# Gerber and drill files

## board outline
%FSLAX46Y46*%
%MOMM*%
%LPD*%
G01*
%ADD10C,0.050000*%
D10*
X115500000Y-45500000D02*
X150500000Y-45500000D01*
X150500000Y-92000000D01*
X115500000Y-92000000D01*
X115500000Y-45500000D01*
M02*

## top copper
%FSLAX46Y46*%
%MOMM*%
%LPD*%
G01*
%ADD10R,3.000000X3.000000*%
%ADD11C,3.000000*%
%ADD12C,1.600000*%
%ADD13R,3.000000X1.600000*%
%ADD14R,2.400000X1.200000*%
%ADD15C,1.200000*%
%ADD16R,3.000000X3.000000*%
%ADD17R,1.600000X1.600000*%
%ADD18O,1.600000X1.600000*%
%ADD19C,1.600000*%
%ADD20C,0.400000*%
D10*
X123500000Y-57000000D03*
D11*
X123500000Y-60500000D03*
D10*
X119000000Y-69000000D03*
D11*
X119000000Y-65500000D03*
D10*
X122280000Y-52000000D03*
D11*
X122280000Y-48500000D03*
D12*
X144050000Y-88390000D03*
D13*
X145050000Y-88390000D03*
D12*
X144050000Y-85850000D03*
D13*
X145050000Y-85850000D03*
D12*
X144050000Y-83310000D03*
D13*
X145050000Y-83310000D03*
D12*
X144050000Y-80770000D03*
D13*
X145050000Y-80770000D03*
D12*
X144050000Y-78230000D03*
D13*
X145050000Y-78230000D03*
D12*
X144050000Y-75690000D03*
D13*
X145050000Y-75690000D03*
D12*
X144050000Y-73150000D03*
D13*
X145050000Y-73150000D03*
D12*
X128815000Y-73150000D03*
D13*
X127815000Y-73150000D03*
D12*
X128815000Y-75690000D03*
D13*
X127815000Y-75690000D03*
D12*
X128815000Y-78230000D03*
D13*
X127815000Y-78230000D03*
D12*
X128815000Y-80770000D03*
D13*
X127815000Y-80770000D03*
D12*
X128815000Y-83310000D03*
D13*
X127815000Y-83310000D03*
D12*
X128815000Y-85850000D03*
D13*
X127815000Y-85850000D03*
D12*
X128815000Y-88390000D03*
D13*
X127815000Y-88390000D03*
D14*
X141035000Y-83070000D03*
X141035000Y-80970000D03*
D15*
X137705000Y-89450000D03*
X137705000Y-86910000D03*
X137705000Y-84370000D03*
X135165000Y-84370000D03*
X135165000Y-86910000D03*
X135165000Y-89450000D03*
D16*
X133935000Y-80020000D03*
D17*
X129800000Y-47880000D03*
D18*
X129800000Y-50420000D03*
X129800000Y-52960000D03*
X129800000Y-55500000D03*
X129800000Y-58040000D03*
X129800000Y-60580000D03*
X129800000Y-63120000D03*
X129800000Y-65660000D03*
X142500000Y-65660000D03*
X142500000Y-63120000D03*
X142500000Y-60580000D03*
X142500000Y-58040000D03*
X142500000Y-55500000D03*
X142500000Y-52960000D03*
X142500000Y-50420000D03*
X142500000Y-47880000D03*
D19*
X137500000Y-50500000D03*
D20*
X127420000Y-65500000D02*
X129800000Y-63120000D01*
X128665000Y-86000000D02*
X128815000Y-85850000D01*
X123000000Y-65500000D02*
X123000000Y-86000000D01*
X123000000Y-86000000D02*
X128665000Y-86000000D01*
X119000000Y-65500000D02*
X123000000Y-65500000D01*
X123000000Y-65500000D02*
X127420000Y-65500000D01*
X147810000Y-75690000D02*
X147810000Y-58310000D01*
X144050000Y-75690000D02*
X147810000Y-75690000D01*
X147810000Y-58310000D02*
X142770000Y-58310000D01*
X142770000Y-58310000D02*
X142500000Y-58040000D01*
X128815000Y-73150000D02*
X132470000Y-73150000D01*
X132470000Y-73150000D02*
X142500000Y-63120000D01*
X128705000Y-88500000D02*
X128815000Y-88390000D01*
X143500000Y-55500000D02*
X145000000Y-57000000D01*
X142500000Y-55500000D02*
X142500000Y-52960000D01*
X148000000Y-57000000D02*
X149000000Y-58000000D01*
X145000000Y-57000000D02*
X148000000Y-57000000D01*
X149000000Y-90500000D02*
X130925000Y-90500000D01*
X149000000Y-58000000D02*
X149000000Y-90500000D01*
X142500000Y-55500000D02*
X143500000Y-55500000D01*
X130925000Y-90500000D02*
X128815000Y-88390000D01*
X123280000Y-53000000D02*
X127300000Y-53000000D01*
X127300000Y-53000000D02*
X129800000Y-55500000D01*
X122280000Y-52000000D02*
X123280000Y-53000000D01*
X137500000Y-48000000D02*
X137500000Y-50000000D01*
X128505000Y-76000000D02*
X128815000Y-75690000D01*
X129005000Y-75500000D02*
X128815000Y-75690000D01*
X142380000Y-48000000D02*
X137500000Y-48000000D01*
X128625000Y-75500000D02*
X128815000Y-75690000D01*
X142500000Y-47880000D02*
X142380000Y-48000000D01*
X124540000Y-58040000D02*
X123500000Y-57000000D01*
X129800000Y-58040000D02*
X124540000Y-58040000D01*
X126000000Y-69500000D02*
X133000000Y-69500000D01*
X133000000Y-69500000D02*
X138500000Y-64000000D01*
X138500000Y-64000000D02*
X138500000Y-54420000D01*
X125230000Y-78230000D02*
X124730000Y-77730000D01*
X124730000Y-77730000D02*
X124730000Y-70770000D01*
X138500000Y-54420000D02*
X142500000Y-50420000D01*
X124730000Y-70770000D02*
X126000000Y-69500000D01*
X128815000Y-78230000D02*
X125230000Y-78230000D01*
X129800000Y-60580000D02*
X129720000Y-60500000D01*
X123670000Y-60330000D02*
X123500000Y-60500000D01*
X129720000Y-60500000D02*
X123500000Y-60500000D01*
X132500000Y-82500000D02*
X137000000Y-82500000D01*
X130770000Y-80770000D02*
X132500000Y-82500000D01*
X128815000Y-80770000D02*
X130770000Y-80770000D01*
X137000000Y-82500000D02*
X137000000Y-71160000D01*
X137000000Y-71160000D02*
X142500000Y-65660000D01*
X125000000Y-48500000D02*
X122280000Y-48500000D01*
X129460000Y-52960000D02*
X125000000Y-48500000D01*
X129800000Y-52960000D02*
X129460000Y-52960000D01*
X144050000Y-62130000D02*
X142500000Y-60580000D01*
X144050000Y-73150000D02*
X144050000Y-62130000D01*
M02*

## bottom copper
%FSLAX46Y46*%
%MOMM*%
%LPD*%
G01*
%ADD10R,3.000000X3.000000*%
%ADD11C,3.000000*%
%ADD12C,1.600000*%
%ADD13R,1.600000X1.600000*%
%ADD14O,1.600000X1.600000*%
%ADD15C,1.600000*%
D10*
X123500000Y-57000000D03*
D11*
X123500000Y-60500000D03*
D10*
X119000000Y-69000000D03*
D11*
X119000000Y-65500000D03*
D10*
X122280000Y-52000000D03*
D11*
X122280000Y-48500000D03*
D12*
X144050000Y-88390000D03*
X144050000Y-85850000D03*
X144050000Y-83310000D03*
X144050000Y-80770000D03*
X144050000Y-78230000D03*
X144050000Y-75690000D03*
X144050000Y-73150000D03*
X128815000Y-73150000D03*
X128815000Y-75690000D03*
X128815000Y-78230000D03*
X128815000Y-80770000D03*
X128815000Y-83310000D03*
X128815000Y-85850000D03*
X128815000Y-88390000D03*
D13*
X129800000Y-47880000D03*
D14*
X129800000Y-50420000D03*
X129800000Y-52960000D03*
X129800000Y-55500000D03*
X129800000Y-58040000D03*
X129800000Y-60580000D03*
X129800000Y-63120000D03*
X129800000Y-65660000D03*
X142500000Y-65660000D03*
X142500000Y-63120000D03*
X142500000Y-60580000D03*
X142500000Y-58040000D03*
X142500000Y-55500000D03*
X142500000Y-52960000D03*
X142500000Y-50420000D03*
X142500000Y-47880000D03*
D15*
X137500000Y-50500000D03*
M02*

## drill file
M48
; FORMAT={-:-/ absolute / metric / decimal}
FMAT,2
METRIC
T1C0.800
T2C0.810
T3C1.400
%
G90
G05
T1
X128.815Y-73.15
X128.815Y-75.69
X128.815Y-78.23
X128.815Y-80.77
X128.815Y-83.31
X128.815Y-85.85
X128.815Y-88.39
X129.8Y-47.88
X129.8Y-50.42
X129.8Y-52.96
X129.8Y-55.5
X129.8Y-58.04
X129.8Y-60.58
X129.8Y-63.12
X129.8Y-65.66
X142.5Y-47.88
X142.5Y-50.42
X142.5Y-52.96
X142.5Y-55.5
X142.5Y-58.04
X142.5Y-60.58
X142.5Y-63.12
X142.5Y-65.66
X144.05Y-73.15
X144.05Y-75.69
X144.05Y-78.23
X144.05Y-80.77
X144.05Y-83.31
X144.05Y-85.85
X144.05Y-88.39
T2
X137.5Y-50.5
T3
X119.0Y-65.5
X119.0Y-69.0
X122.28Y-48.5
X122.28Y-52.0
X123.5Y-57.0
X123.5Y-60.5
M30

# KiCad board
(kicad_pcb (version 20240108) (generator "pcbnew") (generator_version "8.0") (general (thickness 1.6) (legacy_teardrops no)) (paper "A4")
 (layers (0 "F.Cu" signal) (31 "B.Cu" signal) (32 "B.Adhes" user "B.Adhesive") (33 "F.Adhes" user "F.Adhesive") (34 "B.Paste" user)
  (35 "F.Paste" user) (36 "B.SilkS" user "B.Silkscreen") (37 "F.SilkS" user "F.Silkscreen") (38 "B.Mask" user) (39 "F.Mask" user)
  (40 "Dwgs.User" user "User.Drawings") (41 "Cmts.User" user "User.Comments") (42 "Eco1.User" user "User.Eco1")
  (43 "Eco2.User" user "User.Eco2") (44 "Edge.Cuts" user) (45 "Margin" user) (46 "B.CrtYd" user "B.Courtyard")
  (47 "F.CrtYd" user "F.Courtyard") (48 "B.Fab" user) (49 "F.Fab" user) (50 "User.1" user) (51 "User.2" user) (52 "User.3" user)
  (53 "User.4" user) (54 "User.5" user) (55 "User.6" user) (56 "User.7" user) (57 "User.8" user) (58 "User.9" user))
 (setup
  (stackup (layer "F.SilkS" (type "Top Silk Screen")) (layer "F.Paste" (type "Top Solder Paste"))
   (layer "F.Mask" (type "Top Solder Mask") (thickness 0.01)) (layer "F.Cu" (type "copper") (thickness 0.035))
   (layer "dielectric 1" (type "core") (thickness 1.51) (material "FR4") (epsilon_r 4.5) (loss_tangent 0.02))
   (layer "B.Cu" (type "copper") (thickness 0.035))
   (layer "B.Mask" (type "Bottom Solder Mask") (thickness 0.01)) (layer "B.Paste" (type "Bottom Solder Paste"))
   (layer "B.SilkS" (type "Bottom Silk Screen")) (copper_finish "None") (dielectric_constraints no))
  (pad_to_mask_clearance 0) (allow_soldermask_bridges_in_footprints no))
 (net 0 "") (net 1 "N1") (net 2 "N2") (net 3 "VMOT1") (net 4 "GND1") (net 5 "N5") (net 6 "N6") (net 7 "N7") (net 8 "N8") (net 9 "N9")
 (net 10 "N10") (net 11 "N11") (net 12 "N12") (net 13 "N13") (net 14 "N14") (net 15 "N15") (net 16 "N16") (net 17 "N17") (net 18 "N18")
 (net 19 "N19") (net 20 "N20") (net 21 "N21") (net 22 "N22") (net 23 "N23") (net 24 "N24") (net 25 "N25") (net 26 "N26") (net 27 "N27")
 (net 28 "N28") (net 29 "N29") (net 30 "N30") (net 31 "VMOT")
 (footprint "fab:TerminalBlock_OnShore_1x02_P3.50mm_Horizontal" (layer "F.Cu") (at 123.5 57 -90)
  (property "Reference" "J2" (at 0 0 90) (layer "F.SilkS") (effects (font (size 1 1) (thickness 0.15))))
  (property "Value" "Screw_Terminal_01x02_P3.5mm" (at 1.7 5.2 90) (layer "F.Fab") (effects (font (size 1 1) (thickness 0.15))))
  (pad "1" thru_hole rect (at 0 0 270) (size 3 3) (drill 1.4) (layers "*.Cu" "*.Mask") (remove_unused_layers no) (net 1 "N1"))
  (pad "2" thru_hole circle (at 3.5 0 270) (size 3 3) (drill 1.4) (layers "*.Cu" "*.Mask") (remove_unused_layers no) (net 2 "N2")))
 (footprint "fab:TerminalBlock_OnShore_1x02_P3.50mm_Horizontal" (layer "F.Cu") (at 119 69 90)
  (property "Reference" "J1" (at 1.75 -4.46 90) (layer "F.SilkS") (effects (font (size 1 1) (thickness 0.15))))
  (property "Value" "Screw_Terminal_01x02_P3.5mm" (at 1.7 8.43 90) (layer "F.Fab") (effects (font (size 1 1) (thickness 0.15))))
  (pad "1" thru_hole rect (at 0 0 90) (size 3 3) (drill 1.4) (layers "*.Cu" "*.Mask") (remove_unused_layers no) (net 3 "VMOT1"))
  (pad "2" thru_hole circle (at 3.5 0 90) (size 3 3) (drill 1.4) (layers "*.Cu" "*.Mask") (remove_unused_layers no) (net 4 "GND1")))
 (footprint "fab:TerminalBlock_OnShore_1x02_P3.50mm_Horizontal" (layer "F.Cu") (at 122.28 52 90)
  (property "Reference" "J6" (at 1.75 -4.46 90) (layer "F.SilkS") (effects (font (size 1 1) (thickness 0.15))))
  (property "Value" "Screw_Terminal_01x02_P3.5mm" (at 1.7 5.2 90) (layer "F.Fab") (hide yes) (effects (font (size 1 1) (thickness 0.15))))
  (pad "1" thru_hole rect (at 0 0 90) (size 3 3) (drill 1.4) (layers "*.Cu" "*.Mask") (remove_unused_layers no) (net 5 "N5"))
  (pad "2" thru_hole circle (at 3.5 0 90) (size 3 3) (drill 1.4) (layers "*.Cu" "*.Mask") (remove_unused_layers no) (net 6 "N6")))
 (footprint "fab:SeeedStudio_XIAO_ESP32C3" (layer "F.Cu") (at 136.435 80.77 180)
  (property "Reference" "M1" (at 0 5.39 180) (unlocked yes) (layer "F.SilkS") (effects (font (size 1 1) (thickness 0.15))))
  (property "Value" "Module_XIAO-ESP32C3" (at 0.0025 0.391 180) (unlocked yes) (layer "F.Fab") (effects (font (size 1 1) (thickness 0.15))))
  (pad "1" thru_hole circle (at -7.615 -7.62 180) (size 1.6 1.6) (drill 0.8) (layers "*.Cu" "*.Mask") (remove_unused_layers no) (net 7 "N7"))
  (pad "1" smd rect (at -7.615 -7.62 180) (size 3 1.6) (drill (offset -1 0)) (layers "F.Cu" "F.Paste" "F.Mask") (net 7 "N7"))
  (pad "2" thru_hole circle (at -7.615 -5.08 180) (size 1.6 1.6) (drill 0.8) (layers "*.Cu" "*.Mask") (remove_unused_layers no) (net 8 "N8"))
  (pad "2" smd rect (at -7.615 -5.08 180) (size 3 1.6) (drill (offset -1 0)) (layers "F.Cu" "F.Paste" "F.Mask") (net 8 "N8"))
  (pad "3" thru_hole circle (at -7.615 -2.54 180) (size 1.6 1.6) (drill 0.8) (layers "*.Cu" "*.Mask") (remove_unused_layers no) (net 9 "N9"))
  (pad "3" smd rect (at -7.615 -2.54 180) (size 3 1.6) (drill (offset -1 0)) (layers "F.Cu" "F.Paste" "F.Mask") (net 9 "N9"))
  (pad "4" thru_hole circle (at -7.615 0 180) (size 1.6 1.6) (drill 0.8) (layers "*.Cu" "*.Mask") (remove_unused_layers no) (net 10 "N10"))
  (pad "4" smd rect (at -7.615 0 180) (size 3 1.6) (drill (offset -1 0)) (layers "F.Cu" "F.Paste" "F.Mask") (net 10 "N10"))
  (pad "5" thru_hole circle (at -7.615 2.54 180) (size 1.6 1.6) (drill 0.8) (layers "*.Cu" "*.Mask") (remove_unused_layers no)
   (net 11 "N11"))
  (pad "5" smd rect (at -7.615 2.54 180) (size 3 1.6) (drill (offset -1 0)) (layers "F.Cu" "F.Paste" "F.Mask") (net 11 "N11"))
  (pad "6" thru_hole circle (at -7.615 5.08 180) (size 1.6 1.6) (drill 0.8) (layers "*.Cu" "*.Mask") (remove_unused_layers no)
   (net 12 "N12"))
  (pad "6" smd rect (at -7.615 5.08 180) (size 3 1.6) (drill (offset -1 0)) (layers "F.Cu" "F.Paste" "F.Mask") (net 12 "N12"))
  (pad "7" thru_hole circle (at -7.615 7.62 180) (size 1.6 1.6) (drill 0.8) (layers "*.Cu" "*.Mask") (remove_unused_layers no)
   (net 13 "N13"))
  (pad "7" smd rect (at -7.615 7.62 180) (size 3 1.6) (drill (offset -1 0)) (layers "F.Cu" "F.Paste" "F.Mask") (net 13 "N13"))
  (pad "8" thru_hole circle (at 7.62 7.62 180) (size 1.6 1.6) (drill 0.8) (layers "*.Cu" "*.Mask") (remove_unused_layers no) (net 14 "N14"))
  (pad "8" smd rect (at 7.62 7.62 180) (size 3 1.6) (drill (offset 1 0)) (layers "F.Cu" "F.Paste" "F.Mask") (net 14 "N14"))
  (pad "9" thru_hole circle (at 7.62 5.08 180) (size 1.6 1.6) (drill 0.8) (layers "*.Cu" "*.Mask") (remove_unused_layers no) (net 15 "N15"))
  (pad "9" smd rect (at 7.62 5.08 180) (size 3 1.6) (drill (offset 1 0)) (layers "F.Cu" "F.Paste" "F.Mask") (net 15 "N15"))
  (pad "10" thru_hole circle (at 7.62 2.54 180) (size 1.6 1.6) (drill 0.8) (layers "*.Cu" "*.Mask") (remove_unused_layers no) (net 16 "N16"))
  (pad "10" smd rect (at 7.62 2.54 180) (size 3 1.6) (drill (offset 1 0)) (layers "F.Cu" "F.Paste" "F.Mask") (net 16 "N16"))
  (pad "11" thru_hole circle (at 7.62 0 180) (size 1.6 1.6) (drill 0.8) (layers "*.Cu" "*.Mask") (remove_unused_layers no) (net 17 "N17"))
  (pad "11" smd rect (at 7.62 0 180) (size 3 1.6) (drill (offset 1 0)) (layers "F.Cu" "F.Paste" "F.Mask") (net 17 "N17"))
  (pad "12" thru_hole circle (at 7.62 -2.54 180) (size 1.6 1.6) (drill 0.8) (layers "*.Cu" "*.Mask") (remove_unused_layers no)
   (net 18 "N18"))
  (pad "12" smd rect (at 7.62 -2.54 180) (size 3 1.6) (drill (offset 1 0)) (layers "F.Cu" "F.Paste" "F.Mask") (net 18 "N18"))
  (pad "13" thru_hole circle (at 7.62 -5.08 180) (size 1.6 1.6) (drill 0.8) (layers "*.Cu" "*.Mask") (remove_unused_layers no)
   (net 4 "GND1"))
  (pad "13" smd rect (at 7.62 -5.08 180) (size 3 1.6) (drill (offset 1 0)) (layers "F.Cu" "F.Paste" "F.Mask") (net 4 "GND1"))
  (pad "14" thru_hole circle (at 7.62 -7.62 180) (size 1.6 1.6) (drill 0.8) (layers "*.Cu" "*.Mask") (remove_unused_layers no)
   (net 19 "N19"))
  (pad "14" smd rect (at 7.62 -7.62 180) (size 3 1.6) (drill (offset 1 0)) (layers "F.Cu" "F.Paste" "F.Mask") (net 19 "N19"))
  (pad "15" smd rect (at -4.6 -2.3 180) (size 2.4 1.2) (layers "F.Cu" "F.Paste" "F.Mask") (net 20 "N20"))
  (pad "16" smd rect (at -4.6 -0.2 180) (size 2.4 1.2) (layers "F.Cu" "F.Paste" "F.Mask") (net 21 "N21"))
  (pad "17" smd circle (at -1.27 -8.68 180) (size 1.2 1.2) (layers "F.Cu" "F.Paste" "F.Mask") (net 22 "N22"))
  (pad "18" smd circle (at -1.27 -6.14 180) (size 1.2 1.2) (layers "F.Cu" "F.Paste" "F.Mask") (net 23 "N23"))
  (pad "19" smd circle (at -1.27 -3.6 180) (size 1.2 1.2) (layers "F.Cu" "F.Paste" "F.Mask") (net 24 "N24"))
  (pad "20" smd circle (at 1.27 -3.6 180) (size 1.2 1.2) (layers "F.Cu" "F.Paste" "F.Mask") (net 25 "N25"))
  (pad "21" smd circle (at 1.27 -6.14 180) (size 1.2 1.2) (layers "F.Cu" "F.Paste" "F.Mask") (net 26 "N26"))
  (pad "22" smd circle (at 1.27 -8.68 180) (size 1.2 1.2) (layers "F.Cu" "F.Paste" "F.Mask") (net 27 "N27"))
  (pad "23" smd rect (at 2.5 0.75 180) (size 3 3) (layers "F.Cu" "F.Paste" "F.Mask") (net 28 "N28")))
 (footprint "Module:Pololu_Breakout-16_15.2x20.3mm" (layer "F.Cu") (at 129.8 47.88)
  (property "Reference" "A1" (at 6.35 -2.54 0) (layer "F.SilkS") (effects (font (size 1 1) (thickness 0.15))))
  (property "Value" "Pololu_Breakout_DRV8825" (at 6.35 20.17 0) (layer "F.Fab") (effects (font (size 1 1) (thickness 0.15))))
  (pad "1" thru_hole rect (at 0 0) (size 1.6 1.6) (drill oval 0.8) (layers "*.Cu" "*.Mask") (remove_unused_layers no) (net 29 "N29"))
  (pad "2" thru_hole oval (at 0 2.54) (size 1.6 1.6) (drill 0.8) (layers "*.Cu" "*.Mask") (remove_unused_layers no) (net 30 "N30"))
  (pad "3" thru_hole oval (at 0 5.08) (size 1.6 1.6) (drill 0.8) (layers "*.Cu" "*.Mask") (remove_unused_layers no) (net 6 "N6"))
  (pad "4" thru_hole oval (at 0 7.62) (size 1.6 1.6) (drill 0.8) (layers "*.Cu" "*.Mask") (remove_unused_layers no) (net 5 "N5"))
  (pad "5" thru_hole oval (at 0 10.16) (size 1.6 1.6) (drill 0.8) (layers "*.Cu" "*.Mask") (remove_unused_layers no) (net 1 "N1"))
  (pad "6" thru_hole oval (at 0 12.7) (size 1.6 1.6) (drill 0.8) (layers "*.Cu" "*.Mask") (remove_unused_layers no) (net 2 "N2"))
  (pad "7" thru_hole oval (at 0 15.24) (size 1.6 1.6) (drill 0.8) (layers "*.Cu" "*.Mask") (remove_unused_layers no) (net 4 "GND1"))
  (pad "8" thru_hole oval (at 0 17.78) (size 1.6 1.6) (drill 0.8) (layers "*.Cu" "*.Mask") (remove_unused_layers no) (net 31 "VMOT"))
  (pad "9" thru_hole oval (at 12.7 17.78) (size 1.6 1.6) (drill 0.8) (layers "*.Cu" "*.Mask") (remove_unused_layers no) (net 17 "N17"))
  (pad "10" thru_hole oval (at 12.7 15.24) (size 1.6 1.6) (drill 0.8) (layers "*.Cu" "*.Mask") (remove_unused_layers no) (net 14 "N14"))
  (pad "11" thru_hole oval (at 12.7 12.7) (size 1.6 1.6) (drill 0.8) (layers "*.Cu" "*.Mask") (remove_unused_layers no) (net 13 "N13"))
  (pad "12" thru_hole oval (at 12.7 10.16) (size 1.6 1.6) (drill 0.8) (layers "*.Cu" "*.Mask") (remove_unused_layers no) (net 12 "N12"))
  (pad "13" thru_hole oval (at 12.7 7.62) (size 1.6 1.6) (drill 0.8) (layers "*.Cu" "*.Mask") (remove_unused_layers no) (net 19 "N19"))
  (pad "14" thru_hole oval (at 12.7 5.08) (size 1.6 1.6) (drill 0.8) (layers "*.Cu" "*.Mask") (remove_unused_layers no) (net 19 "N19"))
  (pad "15" thru_hole oval (at 12.7 2.54) (size 1.6 1.6) (drill 0.8) (layers "*.Cu" "*.Mask") (remove_unused_layers no) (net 16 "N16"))
  (pad "16" thru_hole oval (at 12.7 0) (size 1.6 1.6) (drill oval 0.8) (layers "*.Cu" "*.Mask") (remove_unused_layers no) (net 15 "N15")))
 (gr_rect (start 115.5 45.5) (end 150.5 92) (stroke (width 0.05) (type default)) (fill none) (layer "Edge.Cuts"))
 (segment (start 127.42 65.5) (end 129.8 63.12) (width 0.4) (layer "F.Cu") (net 4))
 (segment (start 128.665 86) (end 128.815 85.85) (width 0.4) (layer "F.Cu") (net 4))
 (segment (start 123 65.5) (end 123 86) (width 0.4) (layer "F.Cu") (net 4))
 (segment (start 123 86) (end 128.665 86) (width 0.4) (layer "F.Cu") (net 4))
 (segment (start 119 65.5) (end 123 65.5) (width 0.4) (layer "F.Cu") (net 4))
 (segment (start 123 65.5) (end 127.42 65.5) (width 0.4) (layer "F.Cu") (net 4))
 (segment (start 147.81 75.69) (end 147.81 58.31) (width 0.4) (layer "F.Cu") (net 12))
 (segment (start 144.05 75.69) (end 147.81 75.69) (width 0.4) (layer "F.Cu") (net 12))
 (segment (start 147.81 58.31) (end 142.77 58.31) (width 0.4) (layer "F.Cu") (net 12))
 (segment (start 142.77 58.31) (end 142.5 58.04) (width 0.4) (layer "F.Cu") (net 12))
 (segment (start 128.815 73.15) (end 132.47 73.15) (width 0.4) (layer "F.Cu") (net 14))
 (segment (start 132.47 73.15) (end 142.5 63.12) (width 0.4) (layer "F.Cu") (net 14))
 (segment (start 128.705 88.5) (end 128.815 88.39) (width 0.4) (layer "F.Cu") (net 19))
 (segment (start 143.5 55.5) (end 145 57) (width 0.4) (layer "F.Cu") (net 19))
 (segment (start 142.5 55.5) (end 142.5 52.96) (width 0.4) (layer "F.Cu") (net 19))
 (segment (start 148 57) (end 149 58) (width 0.4) (layer "F.Cu") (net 19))
 (segment (start 145 57) (end 148 57) (width 0.4) (layer "F.Cu") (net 19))
 (segment (start 149 90.5) (end 130.925 90.5) (width 0.4) (layer "F.Cu") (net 19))
 (segment (start 149 58) (end 149 90.5) (width 0.4) (layer "F.Cu") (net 19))
 (segment (start 142.5 55.5) (end 143.5 55.5) (width 0.4) (layer "F.Cu") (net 19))
 (segment (start 130.925 90.5) (end 128.815 88.39) (width 0.4) (layer "F.Cu") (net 19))
 (segment (start 123.28 53) (end 127.3 53) (width 0.4) (layer "F.Cu") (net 5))
 (segment (start 127.3 53) (end 129.8 55.5) (width 0.4) (layer "F.Cu") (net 5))
 (segment (start 122.28 52) (end 123.28 53) (width 0.4) (layer "F.Cu") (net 5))
 (segment (start 137.5 48) (end 137.5 50) (width 0.4) (layer "F.Cu") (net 15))
 (segment (start 128.505 76) (end 128.815 75.69) (width 0.4) (layer "F.Cu") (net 15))
 (segment (start 129.005 75.5) (end 128.815 75.69) (width 0.4) (layer "F.Cu") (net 15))
 (segment (start 142.38 48) (end 137.5 48) (width 0.4) (layer "F.Cu") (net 15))
 (segment (start 128.625 75.5) (end 128.815 75.69) (width 0.4) (layer "F.Cu") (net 15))
 (segment (start 142.5 47.88) (end 142.38 48) (width 0.4) (layer "F.Cu") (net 15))
 (via (at 137.5 50.5) (size 1.6) (drill 0.81) (layers "F.Cu" "B.Cu") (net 15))
 (segment (start 124.54 58.04) (end 123.5 57) (width 0.4) (layer "F.Cu") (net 1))
 (segment (start 129.8 58.04) (end 124.54 58.04) (width 0.4) (layer "F.Cu") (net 1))
 (segment (start 126 69.5) (end 133 69.5) (width 0.4) (layer "F.Cu") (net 16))
 (segment (start 133 69.5) (end 138.5 64) (width 0.4) (layer "F.Cu") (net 16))
 (segment (start 138.5 64) (end 138.5 54.42) (width 0.4) (layer "F.Cu") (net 16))
 (segment (start 125.23 78.23) (end 124.73 77.73) (width 0.4) (layer "F.Cu") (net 16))
 (segment (start 124.73 77.73) (end 124.73 70.77) (width 0.4) (layer "F.Cu") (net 16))
 (segment (start 138.5 54.42) (end 142.5 50.42) (width 0.4) (layer "F.Cu") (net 16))
 (segment (start 124.73 70.77) (end 126 69.5) (width 0.4) (layer "F.Cu") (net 16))
 (segment (start 128.815 78.23) (end 125.23 78.23) (width 0.4) (layer "F.Cu") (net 16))
 (segment (start 129.8 60.58) (end 129.72 60.5) (width 0.4) (layer "F.Cu") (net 2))
 (segment (start 123.67 60.33) (end 123.5 60.5) (width 0.4) (layer "F.Cu") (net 2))
 (segment (start 129.72 60.5) (end 123.5 60.5) (width 0.4) (layer "F.Cu") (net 2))
 (segment (start 132.5 82.5) (end 137 82.5) (width 0.4) (layer "F.Cu") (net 17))
 (segment (start 130.77 80.77) (end 132.5 82.5) (width 0.4) (layer "F.Cu") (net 17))
 (segment (start 128.815 80.77) (end 130.77 80.77) (width 0.4) (layer "F.Cu") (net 17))
 (segment (start 137 82.5) (end 137 71.16) (width 0.4) (layer "F.Cu") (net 17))
 (segment (start 137 71.16) (end 142.5 65.66) (width 0.4) (layer "F.Cu") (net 17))
 (segment (start 125 48.5) (end 122.28 48.5) (width 0.4) (layer "F.Cu") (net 6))
 (segment (start 129.46 52.96) (end 125 48.5) (width 0.4) (layer "F.Cu") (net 6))
 (segment (start 129.8 52.96) (end 129.46 52.96) (width 0.4) (layer "F.Cu") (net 6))
 (segment (start 144.05 62.13) (end 142.5 60.58) (width 0.4) (layer "F.Cu") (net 13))
 (segment (start 144.05 73.15) (end 144.05 62.13) (width 0.4) (layer "F.Cu") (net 13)))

